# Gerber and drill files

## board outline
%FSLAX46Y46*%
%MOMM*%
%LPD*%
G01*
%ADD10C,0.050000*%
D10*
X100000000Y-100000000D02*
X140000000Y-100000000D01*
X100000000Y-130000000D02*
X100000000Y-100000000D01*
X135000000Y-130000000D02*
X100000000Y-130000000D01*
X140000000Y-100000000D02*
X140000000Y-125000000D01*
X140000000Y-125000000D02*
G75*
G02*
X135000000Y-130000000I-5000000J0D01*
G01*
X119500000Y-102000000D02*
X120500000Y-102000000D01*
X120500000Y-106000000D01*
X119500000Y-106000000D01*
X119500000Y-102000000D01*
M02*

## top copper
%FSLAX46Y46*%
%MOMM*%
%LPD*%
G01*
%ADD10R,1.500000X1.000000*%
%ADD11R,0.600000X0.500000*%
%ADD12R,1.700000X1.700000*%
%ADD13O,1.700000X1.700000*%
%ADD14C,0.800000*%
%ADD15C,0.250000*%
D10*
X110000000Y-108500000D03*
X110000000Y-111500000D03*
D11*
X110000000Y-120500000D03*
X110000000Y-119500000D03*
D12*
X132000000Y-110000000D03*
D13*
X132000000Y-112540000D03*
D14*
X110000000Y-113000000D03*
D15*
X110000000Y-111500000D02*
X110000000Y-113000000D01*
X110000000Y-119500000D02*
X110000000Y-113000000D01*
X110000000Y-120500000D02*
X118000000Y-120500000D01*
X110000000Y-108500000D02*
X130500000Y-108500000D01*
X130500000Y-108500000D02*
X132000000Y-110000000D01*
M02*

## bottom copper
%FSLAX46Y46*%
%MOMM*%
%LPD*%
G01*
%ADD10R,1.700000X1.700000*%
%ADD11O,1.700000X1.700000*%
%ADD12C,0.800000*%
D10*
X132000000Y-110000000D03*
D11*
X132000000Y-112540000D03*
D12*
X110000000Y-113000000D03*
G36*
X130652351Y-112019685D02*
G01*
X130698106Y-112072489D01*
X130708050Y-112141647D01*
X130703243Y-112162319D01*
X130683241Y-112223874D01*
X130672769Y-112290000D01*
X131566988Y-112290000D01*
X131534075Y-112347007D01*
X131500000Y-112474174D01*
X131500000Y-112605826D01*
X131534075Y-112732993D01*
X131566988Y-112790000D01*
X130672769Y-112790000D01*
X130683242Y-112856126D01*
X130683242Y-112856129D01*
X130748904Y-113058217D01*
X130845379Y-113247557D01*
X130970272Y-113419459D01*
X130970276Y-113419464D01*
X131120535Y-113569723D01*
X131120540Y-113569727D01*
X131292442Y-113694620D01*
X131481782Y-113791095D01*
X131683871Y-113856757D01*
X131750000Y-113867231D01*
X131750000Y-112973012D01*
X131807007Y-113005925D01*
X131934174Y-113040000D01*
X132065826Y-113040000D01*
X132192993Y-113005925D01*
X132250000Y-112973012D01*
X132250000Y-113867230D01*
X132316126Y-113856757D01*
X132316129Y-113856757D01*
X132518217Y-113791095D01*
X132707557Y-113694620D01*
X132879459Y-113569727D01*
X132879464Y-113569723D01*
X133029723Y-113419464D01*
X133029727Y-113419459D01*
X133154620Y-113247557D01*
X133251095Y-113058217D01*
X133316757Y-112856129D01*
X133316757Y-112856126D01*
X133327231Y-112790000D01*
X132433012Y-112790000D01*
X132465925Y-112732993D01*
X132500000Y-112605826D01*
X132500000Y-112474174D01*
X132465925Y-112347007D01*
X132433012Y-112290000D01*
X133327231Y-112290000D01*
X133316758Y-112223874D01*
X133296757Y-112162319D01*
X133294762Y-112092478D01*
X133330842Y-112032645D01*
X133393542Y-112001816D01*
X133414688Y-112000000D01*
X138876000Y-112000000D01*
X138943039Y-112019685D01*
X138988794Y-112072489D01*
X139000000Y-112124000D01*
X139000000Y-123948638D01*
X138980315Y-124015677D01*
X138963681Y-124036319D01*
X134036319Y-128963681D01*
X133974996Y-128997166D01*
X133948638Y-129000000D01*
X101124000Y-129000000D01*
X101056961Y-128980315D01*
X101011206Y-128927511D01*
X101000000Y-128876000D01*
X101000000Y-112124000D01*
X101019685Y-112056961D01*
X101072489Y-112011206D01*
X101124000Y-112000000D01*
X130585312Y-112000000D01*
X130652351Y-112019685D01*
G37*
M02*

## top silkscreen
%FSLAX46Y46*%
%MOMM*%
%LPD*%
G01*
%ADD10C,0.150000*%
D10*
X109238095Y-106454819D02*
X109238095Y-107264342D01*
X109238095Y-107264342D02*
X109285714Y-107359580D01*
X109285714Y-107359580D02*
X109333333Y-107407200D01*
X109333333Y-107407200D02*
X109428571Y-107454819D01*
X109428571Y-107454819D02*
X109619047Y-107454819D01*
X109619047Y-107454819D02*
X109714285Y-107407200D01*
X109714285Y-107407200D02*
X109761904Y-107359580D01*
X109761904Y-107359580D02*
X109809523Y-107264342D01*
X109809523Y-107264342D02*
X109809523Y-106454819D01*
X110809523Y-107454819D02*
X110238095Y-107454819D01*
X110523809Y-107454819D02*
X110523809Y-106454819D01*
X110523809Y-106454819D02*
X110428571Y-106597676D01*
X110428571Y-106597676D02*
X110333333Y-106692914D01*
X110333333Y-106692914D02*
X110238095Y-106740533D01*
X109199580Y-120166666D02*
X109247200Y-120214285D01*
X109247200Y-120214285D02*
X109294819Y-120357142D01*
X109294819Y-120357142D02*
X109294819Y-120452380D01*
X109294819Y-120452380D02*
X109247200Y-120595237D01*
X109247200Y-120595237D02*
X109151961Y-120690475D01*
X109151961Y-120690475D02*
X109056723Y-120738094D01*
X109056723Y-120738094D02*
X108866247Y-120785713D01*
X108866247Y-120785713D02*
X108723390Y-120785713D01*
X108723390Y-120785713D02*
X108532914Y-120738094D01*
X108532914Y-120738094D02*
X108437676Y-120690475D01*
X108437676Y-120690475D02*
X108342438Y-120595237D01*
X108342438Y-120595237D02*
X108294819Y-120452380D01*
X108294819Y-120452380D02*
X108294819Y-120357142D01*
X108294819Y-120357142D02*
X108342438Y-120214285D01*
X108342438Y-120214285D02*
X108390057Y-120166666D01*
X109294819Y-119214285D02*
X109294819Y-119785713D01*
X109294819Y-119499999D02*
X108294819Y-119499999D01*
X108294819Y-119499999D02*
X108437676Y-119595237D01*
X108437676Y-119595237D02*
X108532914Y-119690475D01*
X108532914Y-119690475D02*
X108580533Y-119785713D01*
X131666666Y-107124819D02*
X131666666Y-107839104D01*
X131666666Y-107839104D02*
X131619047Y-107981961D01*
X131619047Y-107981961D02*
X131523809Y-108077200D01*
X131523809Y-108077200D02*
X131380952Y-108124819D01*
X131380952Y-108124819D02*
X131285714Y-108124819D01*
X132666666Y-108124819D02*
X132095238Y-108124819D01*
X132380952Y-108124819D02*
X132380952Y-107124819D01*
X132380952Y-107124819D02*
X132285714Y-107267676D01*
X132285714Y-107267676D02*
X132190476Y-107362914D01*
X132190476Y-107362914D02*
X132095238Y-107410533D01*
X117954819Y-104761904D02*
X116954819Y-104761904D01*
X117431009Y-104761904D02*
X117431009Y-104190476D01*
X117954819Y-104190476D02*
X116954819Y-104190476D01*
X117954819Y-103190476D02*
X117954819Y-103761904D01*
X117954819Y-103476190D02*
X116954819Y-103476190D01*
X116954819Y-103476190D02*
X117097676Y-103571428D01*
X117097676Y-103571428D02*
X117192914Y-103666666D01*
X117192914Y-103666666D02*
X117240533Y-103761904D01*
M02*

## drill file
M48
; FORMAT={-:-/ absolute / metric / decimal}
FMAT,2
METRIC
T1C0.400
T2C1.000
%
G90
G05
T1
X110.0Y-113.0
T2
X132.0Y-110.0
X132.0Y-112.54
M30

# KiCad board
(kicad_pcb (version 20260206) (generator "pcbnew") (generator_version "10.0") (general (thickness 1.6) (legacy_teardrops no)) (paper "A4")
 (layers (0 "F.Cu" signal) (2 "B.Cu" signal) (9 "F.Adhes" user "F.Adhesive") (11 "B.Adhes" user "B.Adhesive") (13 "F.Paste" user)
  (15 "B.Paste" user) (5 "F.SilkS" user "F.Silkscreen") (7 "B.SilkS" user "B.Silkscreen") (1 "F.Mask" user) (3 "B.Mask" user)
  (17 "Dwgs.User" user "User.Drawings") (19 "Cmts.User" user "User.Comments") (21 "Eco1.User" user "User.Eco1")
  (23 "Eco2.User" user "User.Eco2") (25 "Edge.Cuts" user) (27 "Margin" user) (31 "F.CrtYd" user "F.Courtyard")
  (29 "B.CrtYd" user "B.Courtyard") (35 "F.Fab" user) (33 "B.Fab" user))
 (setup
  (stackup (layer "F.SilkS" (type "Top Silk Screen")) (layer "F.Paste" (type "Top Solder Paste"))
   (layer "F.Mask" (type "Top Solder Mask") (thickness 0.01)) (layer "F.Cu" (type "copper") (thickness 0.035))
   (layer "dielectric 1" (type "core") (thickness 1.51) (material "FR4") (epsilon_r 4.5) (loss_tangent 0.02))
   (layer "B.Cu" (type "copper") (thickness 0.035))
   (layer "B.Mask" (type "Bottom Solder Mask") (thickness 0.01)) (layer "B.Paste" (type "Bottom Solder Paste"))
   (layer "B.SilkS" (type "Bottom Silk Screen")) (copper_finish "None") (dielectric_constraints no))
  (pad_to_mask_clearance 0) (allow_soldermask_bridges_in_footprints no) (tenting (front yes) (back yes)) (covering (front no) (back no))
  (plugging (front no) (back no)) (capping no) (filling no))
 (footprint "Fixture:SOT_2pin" (layer "F.Cu") (at 110 110)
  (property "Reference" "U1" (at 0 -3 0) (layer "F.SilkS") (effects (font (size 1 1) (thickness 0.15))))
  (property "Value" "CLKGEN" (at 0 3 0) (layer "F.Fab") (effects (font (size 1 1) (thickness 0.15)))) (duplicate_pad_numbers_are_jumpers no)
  (pad "1" smd rect (at 0 -1.5) (size 1.5 1) (layers "F.Cu" "F.Mask" "F.Paste") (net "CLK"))
  (pad "2" smd rect (at 0 1.5) (size 1.5 1) (layers "F.Cu" "F.Mask" "F.Paste") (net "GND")))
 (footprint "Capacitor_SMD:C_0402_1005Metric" (layer "F.Cu") (at 110 120 90)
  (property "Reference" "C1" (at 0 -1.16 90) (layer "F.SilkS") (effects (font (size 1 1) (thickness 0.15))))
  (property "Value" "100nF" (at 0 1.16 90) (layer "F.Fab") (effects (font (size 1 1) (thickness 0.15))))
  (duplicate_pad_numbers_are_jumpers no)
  (pad "1" smd rect (at -0.5 0 90) (size 0.5 0.6) (layers "F.Cu" "F.Mask" "F.Paste") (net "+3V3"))
  (pad "2" smd rect (at 0.5 0 90) (size 0.5 0.6) (layers "F.Cu" "F.Mask" "F.Paste") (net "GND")))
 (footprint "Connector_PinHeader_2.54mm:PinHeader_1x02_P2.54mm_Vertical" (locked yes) (layer "F.Cu") (at 132 110)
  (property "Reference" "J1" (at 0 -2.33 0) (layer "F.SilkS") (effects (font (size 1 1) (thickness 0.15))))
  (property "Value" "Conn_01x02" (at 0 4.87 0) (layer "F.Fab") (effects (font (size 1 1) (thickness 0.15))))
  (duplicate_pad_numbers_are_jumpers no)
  (pad "1" thru_hole rect (at 0 0) (size 1.7 1.7) (drill 1) (layers "*.Cu" "*.Mask") (remove_unused_layers no) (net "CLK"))
  (pad "2" thru_hole oval (at 0 2.54) (size 1.7 1.7) (drill 1) (layers "*.Cu" "*.Mask") (remove_unused_layers no) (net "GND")))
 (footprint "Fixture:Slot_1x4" (layer "F.Cu") (at 120 104 90)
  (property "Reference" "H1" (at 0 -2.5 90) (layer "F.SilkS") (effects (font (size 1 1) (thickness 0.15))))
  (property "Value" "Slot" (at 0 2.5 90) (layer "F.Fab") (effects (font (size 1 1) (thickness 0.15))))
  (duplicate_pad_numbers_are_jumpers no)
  (fp_rect (start -2 -0.5) (end 2 0.5) (stroke (width 0.05) (type default)) (fill no) (layer "Edge.Cuts")))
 (gr_line (start 100 100) (end 140 100) (stroke (width 0.05) (type default)) (layer "Edge.Cuts"))
 (gr_line (start 100 130) (end 100 100) (stroke (width 0.05) (type default)) (layer "Edge.Cuts"))
 (gr_line (start 135 130) (end 100 130) (stroke (width 0.05) (type default)) (layer "Edge.Cuts"))
 (gr_line (start 140 100) (end 140 125) (stroke (width 0.05) (type default)) (layer "Edge.Cuts"))
 (gr_arc (start 140 125) (mid 138.535534 128.535534) (end 135 130) (stroke (width 0.05) (type default)) (layer "Edge.Cuts"))
 (segment (start 110 111.5) (end 110 113) (width 0.25) (layer "F.Cu") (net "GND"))
 (segment (start 110 119.5) (end 110 113) (width 0.25) (layer "F.Cu") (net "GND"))
 (via (at 110 113) (size 0.8) (drill 0.4) (layers "F.Cu" "B.Cu") (capping no) (covering (front no) (back no))
  (plugging (front no) (back no)) (filling no) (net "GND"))
 (segment (start 110 120.5) (end 118 120.5) (width 0.25) (layer "F.Cu") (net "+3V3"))
 (segment (start 110 108.5) (end 130.5 108.5) (width 0.25) (layer "F.Cu") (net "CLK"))
 (segment (start 130.5 108.5) (end 132 110) (width 0.25) (layer "F.Cu") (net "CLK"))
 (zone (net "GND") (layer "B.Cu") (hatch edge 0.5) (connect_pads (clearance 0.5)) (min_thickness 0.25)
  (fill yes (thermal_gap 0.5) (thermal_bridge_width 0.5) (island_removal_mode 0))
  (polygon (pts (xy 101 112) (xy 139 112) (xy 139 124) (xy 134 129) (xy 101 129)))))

